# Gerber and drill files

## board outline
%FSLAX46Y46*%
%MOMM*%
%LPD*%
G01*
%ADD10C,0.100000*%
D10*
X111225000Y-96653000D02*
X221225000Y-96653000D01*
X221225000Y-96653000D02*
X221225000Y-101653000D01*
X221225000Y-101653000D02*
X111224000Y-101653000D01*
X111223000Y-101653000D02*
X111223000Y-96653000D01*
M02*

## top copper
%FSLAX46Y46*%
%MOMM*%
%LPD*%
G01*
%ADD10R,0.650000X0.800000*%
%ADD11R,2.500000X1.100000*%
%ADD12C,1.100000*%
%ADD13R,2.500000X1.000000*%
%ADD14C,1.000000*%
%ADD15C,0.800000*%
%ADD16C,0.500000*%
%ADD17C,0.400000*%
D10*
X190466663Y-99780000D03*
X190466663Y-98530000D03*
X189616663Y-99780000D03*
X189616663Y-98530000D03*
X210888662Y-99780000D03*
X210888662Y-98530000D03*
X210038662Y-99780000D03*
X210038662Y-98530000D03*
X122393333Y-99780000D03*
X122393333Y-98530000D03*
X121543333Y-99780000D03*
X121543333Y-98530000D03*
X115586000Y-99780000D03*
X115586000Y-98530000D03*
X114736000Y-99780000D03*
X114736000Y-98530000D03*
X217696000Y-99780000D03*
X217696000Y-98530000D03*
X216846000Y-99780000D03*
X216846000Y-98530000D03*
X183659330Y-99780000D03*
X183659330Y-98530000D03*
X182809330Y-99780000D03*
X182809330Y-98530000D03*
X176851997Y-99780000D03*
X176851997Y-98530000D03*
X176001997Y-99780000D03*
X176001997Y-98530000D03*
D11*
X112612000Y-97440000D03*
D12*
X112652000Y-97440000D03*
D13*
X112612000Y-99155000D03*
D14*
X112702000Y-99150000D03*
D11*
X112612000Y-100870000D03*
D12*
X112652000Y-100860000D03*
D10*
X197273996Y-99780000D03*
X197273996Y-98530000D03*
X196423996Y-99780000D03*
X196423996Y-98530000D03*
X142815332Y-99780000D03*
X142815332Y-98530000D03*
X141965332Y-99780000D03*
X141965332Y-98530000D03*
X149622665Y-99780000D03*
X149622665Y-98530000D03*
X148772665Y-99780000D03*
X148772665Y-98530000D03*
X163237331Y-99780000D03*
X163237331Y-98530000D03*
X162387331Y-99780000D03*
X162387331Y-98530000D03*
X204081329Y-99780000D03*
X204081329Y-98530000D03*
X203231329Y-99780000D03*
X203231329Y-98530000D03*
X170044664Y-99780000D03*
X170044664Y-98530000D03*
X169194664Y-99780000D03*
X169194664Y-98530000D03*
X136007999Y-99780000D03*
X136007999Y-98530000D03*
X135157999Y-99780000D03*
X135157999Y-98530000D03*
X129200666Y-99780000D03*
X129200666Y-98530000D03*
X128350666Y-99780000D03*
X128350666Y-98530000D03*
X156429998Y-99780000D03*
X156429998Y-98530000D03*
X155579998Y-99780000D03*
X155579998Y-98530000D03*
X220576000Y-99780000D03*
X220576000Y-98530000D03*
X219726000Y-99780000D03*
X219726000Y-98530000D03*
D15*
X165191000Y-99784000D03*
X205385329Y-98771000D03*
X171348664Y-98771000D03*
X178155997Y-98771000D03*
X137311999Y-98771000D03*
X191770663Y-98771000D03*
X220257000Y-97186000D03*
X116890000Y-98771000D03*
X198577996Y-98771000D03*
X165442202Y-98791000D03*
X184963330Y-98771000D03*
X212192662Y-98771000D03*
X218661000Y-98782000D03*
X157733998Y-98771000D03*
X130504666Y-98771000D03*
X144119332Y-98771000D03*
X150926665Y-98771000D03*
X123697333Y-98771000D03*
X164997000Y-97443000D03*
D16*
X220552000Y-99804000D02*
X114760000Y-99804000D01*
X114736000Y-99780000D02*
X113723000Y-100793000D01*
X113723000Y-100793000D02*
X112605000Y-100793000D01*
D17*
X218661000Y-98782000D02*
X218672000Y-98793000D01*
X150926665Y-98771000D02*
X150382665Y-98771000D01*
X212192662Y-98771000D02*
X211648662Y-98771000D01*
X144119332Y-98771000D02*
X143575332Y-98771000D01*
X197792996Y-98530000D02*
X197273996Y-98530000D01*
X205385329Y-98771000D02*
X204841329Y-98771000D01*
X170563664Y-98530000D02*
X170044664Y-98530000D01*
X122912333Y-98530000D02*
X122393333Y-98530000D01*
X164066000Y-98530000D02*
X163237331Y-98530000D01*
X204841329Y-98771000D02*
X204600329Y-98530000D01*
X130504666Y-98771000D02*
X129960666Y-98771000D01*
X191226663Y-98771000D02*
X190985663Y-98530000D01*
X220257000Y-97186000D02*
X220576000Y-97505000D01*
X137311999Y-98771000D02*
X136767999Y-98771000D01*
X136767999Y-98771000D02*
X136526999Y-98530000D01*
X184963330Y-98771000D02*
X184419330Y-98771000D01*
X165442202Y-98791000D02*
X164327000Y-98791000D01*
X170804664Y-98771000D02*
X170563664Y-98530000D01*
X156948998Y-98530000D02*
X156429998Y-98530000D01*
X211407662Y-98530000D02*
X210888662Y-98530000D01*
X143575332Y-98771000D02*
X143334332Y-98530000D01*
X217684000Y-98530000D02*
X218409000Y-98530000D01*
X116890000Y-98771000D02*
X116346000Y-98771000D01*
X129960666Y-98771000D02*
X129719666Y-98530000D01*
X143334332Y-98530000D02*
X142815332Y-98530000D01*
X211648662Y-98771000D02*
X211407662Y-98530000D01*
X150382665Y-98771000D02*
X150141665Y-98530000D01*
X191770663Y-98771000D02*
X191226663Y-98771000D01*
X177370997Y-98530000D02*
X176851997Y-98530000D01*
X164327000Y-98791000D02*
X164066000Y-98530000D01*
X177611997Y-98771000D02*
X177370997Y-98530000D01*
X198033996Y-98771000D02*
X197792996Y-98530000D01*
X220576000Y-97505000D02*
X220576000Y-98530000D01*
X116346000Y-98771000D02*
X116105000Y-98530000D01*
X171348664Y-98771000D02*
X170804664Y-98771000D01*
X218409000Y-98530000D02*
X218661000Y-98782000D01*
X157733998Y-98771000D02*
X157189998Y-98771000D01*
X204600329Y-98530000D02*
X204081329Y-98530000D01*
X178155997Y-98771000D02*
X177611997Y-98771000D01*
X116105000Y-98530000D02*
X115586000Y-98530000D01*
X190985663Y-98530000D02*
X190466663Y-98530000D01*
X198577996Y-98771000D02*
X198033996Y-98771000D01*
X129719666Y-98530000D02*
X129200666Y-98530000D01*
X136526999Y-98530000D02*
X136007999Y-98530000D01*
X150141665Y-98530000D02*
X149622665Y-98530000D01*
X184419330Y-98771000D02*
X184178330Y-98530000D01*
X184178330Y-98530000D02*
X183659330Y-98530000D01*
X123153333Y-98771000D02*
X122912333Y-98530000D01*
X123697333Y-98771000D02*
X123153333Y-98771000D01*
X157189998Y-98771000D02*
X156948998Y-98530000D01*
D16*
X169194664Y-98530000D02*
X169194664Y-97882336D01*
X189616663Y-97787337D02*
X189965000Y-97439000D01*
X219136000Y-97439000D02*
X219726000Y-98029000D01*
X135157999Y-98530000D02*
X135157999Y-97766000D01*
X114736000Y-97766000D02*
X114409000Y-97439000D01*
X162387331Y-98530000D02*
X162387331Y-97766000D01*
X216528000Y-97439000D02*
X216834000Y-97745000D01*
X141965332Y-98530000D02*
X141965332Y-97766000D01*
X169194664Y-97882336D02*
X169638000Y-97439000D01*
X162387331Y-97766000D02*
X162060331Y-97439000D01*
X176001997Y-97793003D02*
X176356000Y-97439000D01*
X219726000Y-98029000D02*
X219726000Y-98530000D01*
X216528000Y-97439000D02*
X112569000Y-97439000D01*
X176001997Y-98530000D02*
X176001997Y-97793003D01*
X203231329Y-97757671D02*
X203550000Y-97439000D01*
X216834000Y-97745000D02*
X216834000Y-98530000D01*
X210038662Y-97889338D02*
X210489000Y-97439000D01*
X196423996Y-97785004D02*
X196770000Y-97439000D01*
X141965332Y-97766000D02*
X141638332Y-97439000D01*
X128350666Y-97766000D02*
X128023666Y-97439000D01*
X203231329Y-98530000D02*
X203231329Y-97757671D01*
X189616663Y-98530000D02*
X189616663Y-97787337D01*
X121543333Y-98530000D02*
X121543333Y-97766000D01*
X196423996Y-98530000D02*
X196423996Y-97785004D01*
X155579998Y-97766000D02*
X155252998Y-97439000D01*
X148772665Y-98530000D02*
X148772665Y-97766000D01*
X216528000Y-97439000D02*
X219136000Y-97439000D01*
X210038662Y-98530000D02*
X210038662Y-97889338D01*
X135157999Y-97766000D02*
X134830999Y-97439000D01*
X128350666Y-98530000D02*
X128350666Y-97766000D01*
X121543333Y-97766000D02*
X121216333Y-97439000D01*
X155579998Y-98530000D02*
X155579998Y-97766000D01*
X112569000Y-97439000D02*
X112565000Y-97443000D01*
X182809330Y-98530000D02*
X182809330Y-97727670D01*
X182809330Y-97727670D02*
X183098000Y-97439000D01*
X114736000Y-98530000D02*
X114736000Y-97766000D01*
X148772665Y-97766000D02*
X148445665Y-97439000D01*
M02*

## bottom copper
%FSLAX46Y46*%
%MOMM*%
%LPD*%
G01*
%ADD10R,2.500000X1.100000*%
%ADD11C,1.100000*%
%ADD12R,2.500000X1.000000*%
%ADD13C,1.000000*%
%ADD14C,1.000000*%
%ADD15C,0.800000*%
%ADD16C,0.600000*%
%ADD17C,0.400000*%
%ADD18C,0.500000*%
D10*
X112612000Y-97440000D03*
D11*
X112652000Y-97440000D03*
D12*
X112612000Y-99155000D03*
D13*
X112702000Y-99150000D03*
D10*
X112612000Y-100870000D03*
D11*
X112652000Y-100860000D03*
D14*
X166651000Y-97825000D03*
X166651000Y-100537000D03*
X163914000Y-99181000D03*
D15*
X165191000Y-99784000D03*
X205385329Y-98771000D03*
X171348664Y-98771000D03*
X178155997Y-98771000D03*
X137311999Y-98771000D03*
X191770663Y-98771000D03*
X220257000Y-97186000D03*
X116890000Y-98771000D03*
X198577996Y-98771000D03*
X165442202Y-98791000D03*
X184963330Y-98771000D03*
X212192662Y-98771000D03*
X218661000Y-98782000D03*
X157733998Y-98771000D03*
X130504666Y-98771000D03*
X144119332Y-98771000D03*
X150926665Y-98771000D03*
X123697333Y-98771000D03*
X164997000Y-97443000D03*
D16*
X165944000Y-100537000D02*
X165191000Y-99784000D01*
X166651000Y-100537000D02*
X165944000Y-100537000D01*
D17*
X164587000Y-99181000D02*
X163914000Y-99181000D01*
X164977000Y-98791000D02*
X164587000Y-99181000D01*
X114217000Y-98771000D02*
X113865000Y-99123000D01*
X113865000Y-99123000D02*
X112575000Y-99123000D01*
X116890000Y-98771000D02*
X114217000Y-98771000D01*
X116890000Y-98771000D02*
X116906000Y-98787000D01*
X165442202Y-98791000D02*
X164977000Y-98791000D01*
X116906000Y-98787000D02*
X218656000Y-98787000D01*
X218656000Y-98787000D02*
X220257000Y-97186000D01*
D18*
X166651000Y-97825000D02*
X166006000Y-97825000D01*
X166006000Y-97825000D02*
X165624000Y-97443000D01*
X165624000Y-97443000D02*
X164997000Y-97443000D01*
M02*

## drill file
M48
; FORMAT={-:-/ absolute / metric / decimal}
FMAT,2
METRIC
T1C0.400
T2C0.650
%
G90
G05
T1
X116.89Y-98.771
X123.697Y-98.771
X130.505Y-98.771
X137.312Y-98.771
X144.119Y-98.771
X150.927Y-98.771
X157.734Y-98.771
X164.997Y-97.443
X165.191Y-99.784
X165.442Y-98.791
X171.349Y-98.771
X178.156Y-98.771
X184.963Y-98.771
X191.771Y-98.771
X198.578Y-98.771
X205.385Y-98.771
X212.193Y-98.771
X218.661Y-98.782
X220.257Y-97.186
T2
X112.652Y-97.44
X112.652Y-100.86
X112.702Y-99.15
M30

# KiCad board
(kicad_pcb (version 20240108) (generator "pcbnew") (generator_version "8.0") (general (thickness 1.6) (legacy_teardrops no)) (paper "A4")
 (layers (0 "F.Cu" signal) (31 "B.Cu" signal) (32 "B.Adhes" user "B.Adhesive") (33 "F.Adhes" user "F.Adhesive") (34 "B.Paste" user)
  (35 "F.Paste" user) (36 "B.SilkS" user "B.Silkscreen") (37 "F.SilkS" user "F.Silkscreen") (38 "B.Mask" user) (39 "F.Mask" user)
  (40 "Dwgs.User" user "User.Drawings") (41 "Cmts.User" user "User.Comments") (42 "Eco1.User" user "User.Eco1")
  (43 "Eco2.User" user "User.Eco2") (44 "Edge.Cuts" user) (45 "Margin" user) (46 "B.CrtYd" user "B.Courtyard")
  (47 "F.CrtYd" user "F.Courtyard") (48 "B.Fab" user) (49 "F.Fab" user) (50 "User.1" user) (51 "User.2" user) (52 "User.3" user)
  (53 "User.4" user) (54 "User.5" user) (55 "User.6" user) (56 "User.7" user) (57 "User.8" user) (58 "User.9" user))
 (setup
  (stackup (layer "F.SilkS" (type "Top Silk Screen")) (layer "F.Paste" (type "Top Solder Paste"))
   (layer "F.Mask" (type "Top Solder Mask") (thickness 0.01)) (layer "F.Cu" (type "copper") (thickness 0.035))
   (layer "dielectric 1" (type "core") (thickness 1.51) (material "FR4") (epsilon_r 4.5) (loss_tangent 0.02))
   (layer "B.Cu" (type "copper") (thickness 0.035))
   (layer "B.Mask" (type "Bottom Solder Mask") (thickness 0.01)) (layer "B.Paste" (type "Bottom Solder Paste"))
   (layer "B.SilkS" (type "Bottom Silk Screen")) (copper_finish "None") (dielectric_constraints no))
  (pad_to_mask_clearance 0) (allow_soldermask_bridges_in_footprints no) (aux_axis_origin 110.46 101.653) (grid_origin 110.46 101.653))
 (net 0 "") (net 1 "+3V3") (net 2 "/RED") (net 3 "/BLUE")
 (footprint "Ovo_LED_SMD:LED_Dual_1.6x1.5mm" (layer "F.Cu") (at 190.041663 99.155 90)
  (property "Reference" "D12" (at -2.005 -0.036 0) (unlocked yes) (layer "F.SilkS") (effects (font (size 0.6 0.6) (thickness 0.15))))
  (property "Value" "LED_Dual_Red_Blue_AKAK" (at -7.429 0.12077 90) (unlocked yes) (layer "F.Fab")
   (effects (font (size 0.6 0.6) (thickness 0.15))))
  (pad "1" smd rect (at -0.625 0.425 90) (size 0.8 0.65) (layers "F.Cu" "F.Paste" "F.Mask") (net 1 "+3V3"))
  (pad "2" smd rect (at 0.625 0.425 90) (size 0.8 0.65) (layers "F.Cu" "F.Paste" "F.Mask") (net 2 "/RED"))
  (pad "3" smd rect (at -0.625 -0.425 90) (size 0.8 0.65) (layers "F.Cu" "F.Paste" "F.Mask") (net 1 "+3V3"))
  (pad "4" smd rect (at 0.625 -0.425 90) (size 0.8 0.65) (layers "F.Cu" "F.Paste" "F.Mask") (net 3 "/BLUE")))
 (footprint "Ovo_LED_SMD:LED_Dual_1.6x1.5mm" (layer "F.Cu") (at 210.463662 99.155 90)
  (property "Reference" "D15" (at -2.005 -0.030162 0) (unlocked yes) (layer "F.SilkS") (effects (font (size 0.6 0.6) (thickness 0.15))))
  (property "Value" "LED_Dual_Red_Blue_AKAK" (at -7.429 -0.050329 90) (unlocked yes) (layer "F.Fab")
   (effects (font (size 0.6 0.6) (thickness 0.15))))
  (pad "1" smd rect (at -0.625 0.425 90) (size 0.8 0.65) (layers "F.Cu" "F.Paste" "F.Mask") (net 1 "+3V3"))
  (pad "2" smd rect (at 0.625 0.425 90) (size 0.8 0.65) (layers "F.Cu" "F.Paste" "F.Mask") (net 2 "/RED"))
  (pad "3" smd rect (at -0.625 -0.425 90) (size 0.8 0.65) (layers "F.Cu" "F.Paste" "F.Mask") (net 1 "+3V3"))
  (pad "4" smd rect (at 0.625 -0.425 90) (size 0.8 0.65) (layers "F.Cu" "F.Paste" "F.Mask") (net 3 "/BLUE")))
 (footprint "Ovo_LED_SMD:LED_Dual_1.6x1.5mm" (layer "F.Cu") (at 121.968333 99.155 90)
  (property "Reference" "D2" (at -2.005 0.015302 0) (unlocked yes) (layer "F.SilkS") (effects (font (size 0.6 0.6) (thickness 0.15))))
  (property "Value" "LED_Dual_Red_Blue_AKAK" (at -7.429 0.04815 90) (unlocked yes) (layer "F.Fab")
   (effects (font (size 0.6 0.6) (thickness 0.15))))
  (pad "1" smd rect (at -0.625 0.425 90) (size 0.8 0.65) (layers "F.Cu" "F.Paste" "F.Mask") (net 1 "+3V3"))
  (pad "2" smd rect (at 0.625 0.425 90) (size 0.8 0.65) (layers "F.Cu" "F.Paste" "F.Mask") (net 2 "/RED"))
  (pad "3" smd rect (at -0.625 -0.425 90) (size 0.8 0.65) (layers "F.Cu" "F.Paste" "F.Mask") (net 1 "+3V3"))
  (pad "4" smd rect (at 0.625 -0.425 90) (size 0.8 0.65) (layers "F.Cu" "F.Paste" "F.Mask") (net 3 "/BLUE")))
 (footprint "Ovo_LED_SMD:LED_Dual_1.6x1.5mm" (layer "F.Cu") (at 115.161 99.155 90)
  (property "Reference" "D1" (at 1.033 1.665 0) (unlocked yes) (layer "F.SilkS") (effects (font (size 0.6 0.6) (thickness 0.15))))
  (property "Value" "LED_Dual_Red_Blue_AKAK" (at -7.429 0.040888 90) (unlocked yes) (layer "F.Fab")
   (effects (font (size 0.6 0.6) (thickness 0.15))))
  (pad "1" smd rect (at -0.625 0.425 90) (size 0.8 0.65) (layers "F.Cu" "F.Paste" "F.Mask") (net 1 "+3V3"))
  (pad "2" smd rect (at 0.625 0.425 90) (size 0.8 0.65) (layers "F.Cu" "F.Paste" "F.Mask") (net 2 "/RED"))
  (pad "3" smd rect (at -0.625 -0.425 90) (size 0.8 0.65) (layers "F.Cu" "F.Paste" "F.Mask") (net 1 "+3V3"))
  (pad "4" smd rect (at 0.625 -0.425 90) (size 0.8 0.65) (layers "F.Cu" "F.Paste" "F.Mask") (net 3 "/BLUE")))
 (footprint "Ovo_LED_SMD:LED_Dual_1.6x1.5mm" (layer "F.Cu") (at 217.271 99.155 90)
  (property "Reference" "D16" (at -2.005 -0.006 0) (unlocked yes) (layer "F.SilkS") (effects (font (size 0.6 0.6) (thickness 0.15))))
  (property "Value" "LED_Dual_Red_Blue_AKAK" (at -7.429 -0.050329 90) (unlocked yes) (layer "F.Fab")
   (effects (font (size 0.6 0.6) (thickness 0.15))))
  (pad "1" smd rect (at -0.625 0.425 90) (size 0.8 0.65) (layers "F.Cu" "F.Paste" "F.Mask") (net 1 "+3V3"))
  (pad "2" smd rect (at 0.625 0.425 90) (size 0.8 0.65) (layers "F.Cu" "F.Paste" "F.Mask") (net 2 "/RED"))
  (pad "3" smd rect (at -0.625 -0.425 90) (size 0.8 0.65) (layers "F.Cu" "F.Paste" "F.Mask") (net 1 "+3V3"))
  (pad "4" smd rect (at 0.625 -0.425 90) (size 0.8 0.65) (layers "F.Cu" "F.Paste" "F.Mask") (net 3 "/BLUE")))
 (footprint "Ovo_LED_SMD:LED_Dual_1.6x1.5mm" (layer "F.Cu") (at 183.23433 99.155 90)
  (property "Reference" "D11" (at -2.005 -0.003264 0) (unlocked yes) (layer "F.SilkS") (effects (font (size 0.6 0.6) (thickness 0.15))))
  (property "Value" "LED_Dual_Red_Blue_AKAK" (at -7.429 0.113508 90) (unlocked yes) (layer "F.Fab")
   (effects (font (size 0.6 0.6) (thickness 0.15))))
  (pad "1" smd rect (at -0.625 0.425 90) (size 0.8 0.65) (layers "F.Cu" "F.Paste" "F.Mask") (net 1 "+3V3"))
  (pad "2" smd rect (at 0.625 0.425 90) (size 0.8 0.65) (layers "F.Cu" "F.Paste" "F.Mask") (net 2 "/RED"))
  (pad "3" smd rect (at -0.625 -0.425 90) (size 0.8 0.65) (layers "F.Cu" "F.Paste" "F.Mask") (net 1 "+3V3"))
  (pad "4" smd rect (at 0.625 -0.425 90) (size 0.8 0.65) (layers "F.Cu" "F.Paste" "F.Mask") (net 3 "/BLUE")))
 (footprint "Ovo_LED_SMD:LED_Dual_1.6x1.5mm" (layer "F.Cu") (at 176.426997 99.155 90)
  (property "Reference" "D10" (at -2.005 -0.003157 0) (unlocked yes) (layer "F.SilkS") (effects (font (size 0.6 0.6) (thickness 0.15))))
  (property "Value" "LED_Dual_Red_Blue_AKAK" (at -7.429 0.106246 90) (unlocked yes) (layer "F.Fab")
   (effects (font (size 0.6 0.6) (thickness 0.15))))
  (pad "1" smd rect (at -0.625 0.425 90) (size 0.8 0.65) (layers "F.Cu" "F.Paste" "F.Mask") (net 1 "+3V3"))
  (pad "2" smd rect (at 0.625 0.425 90) (size 0.8 0.65) (layers "F.Cu" "F.Paste" "F.Mask") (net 2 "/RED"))
  (pad "3" smd rect (at -0.625 -0.425 90) (size 0.8 0.65) (layers "F.Cu" "F.Paste" "F.Mask") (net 1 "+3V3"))
  (pad "4" smd rect (at 0.625 -0.425 90) (size 0.8 0.65) (layers "F.Cu" "F.Paste" "F.Mask") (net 3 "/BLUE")))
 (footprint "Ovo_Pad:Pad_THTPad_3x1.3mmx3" (layer "F.Cu") (at 112.652 97.52)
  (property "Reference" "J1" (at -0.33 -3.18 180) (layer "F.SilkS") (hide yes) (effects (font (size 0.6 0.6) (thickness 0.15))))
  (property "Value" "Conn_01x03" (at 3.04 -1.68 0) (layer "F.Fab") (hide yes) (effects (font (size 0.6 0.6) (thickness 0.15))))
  (pad "1" smd rect (at -0.04 -0.08 180) (size 2.5 1.1) (layers "F.Cu" "F.Paste" "F.Mask") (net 3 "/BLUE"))
  (pad "1" smd rect (at -0.04 -0.08 180) (size 2.5 1.1) (layers "B.Cu" "B.Paste" "B.Mask") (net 3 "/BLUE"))
  (pad "1" thru_hole circle (at 0 -0.08) (size 1.1 1.1) (drill 0.65) (layers "*.Cu" "*.Mask") (remove_unused_layers no) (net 3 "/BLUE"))
  (pad "2" smd rect (at -0.04 1.635 180) (size 2.5 1) (layers "F.Cu" "F.Paste" "F.Mask") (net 2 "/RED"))
  (pad "2" smd rect (at -0.04 1.635 180) (size 2.5 1) (layers "B.Cu" "B.Paste" "B.Mask") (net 2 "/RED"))
  (pad "2" thru_hole circle (at 0.05 1.63) (size 1 1) (drill 0.65) (layers "*.Cu" "*.Mask") (remove_unused_layers no) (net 2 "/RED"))
  (pad "3" smd rect (at -0.04 3.35 180) (size 2.5 1.1) (layers "F.Cu" "F.Paste" "F.Mask") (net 1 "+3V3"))
  (pad "3" smd rect (at -0.04 3.35 180) (size 2.5 1.1) (layers "B.Cu" "B.Paste" "B.Mask") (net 1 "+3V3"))
  (pad "3" thru_hole circle (at 0 3.34) (size 1.1 1.1) (drill 0.65) (layers "*.Cu" "*.Mask") (remove_unused_layers no) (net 1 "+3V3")))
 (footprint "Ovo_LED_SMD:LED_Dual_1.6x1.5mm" (layer "F.Cu") (at 196.848996 99.155 90)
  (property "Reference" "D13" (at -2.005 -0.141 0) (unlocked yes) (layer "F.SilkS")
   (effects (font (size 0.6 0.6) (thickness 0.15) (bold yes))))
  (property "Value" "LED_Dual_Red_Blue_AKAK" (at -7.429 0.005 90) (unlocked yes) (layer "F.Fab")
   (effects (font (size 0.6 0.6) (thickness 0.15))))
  (pad "1" smd rect (at -0.625 0.425 90) (size 0.8 0.65) (layers "F.Cu" "F.Paste" "F.Mask") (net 1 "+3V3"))
  (pad "2" smd rect (at 0.625 0.425 90) (size 0.8 0.65) (layers "F.Cu" "F.Paste" "F.Mask") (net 2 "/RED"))
  (pad "3" smd rect (at -0.625 -0.425 90) (size 0.8 0.65) (layers "F.Cu" "F.Paste" "F.Mask") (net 1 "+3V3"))
  (pad "4" smd rect (at 0.625 -0.425 90) (size 0.8 0.65) (layers "F.Cu" "F.Paste" "F.Mask") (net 3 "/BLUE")))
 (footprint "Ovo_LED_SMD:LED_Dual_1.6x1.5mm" (layer "F.Cu") (at 142.390332 99.155 90)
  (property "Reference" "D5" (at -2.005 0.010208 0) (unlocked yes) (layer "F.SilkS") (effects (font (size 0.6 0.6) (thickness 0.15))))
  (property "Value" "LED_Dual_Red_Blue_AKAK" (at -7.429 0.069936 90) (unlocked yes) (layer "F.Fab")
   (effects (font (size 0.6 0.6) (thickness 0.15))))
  (pad "1" smd rect (at -0.625 0.425 90) (size 0.8 0.65) (layers "F.Cu" "F.Paste" "F.Mask") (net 1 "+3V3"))
  (pad "2" smd rect (at 0.625 0.425 90) (size 0.8 0.65) (layers "F.Cu" "F.Paste" "F.Mask") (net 2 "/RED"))
  (pad "3" smd rect (at -0.625 -0.425 90) (size 0.8 0.65) (layers "F.Cu" "F.Paste" "F.Mask") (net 1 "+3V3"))
  (pad "4" smd rect (at 0.625 -0.425 90) (size 0.8 0.65) (layers "F.Cu" "F.Paste" "F.Mask") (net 3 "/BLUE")))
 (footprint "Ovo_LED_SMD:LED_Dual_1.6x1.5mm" (layer "F.Cu") (at 149.197665 99.155 90)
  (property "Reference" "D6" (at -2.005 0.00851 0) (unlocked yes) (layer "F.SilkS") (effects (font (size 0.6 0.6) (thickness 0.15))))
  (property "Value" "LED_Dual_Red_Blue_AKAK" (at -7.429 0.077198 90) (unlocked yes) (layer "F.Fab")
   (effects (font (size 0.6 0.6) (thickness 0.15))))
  (pad "1" smd rect (at -0.625 0.425 90) (size 0.8 0.65) (layers "F.Cu" "F.Paste" "F.Mask") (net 1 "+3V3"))
  (pad "2" smd rect (at 0.625 0.425 90) (size 0.8 0.65) (layers "F.Cu" "F.Paste" "F.Mask") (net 2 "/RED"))
  (pad "3" smd rect (at -0.625 -0.425 90) (size 0.8 0.65) (layers "F.Cu" "F.Paste" "F.Mask") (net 1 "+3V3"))
  (pad "4" smd rect (at 0.625 -0.425 90) (size 0.8 0.65) (layers "F.Cu" "F.Paste" "F.Mask") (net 3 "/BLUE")))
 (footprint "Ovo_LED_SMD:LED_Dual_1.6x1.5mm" (layer "F.Cu") (at 162.812331 99.155 90)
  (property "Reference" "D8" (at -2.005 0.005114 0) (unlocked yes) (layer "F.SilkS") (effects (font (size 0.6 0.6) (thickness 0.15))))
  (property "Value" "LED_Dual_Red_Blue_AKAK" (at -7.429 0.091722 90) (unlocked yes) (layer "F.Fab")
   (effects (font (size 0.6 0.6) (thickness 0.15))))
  (pad "1" smd rect (at -0.625 0.425 90) (size 0.8 0.65) (layers "F.Cu" "F.Paste" "F.Mask") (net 1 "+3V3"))
  (pad "2" smd rect (at 0.625 0.425 90) (size 0.8 0.65) (layers "F.Cu" "F.Paste" "F.Mask") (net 2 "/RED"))
  (pad "3" smd rect (at -0.625 -0.425 90) (size 0.8 0.65) (layers "F.Cu" "F.Paste" "F.Mask") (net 1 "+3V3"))
  (pad "4" smd rect (at 0.625 -0.425 90) (size 0.8 0.65) (layers "F.Cu" "F.Paste" "F.Mask") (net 3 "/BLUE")))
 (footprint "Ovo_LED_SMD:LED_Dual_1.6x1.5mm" (layer "F.Cu") (at 203.656329 99.155 90)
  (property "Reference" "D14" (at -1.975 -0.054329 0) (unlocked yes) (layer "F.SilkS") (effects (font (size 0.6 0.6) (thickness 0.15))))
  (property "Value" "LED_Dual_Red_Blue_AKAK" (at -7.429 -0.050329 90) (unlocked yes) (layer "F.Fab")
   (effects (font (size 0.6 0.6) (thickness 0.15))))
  (pad "1" smd rect (at -0.625 0.425 90) (size 0.8 0.65) (layers "F.Cu" "F.Paste" "F.Mask") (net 1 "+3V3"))
  (pad "2" smd rect (at 0.625 0.425 90) (size 0.8 0.65) (layers "F.Cu" "F.Paste" "F.Mask") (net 2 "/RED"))
  (pad "3" smd rect (at -0.625 -0.425 90) (size 0.8 0.65) (layers "F.Cu" "F.Paste" "F.Mask") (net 1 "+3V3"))
  (pad "4" smd rect (at 0.625 -0.425 90) (size 0.8 0.65) (layers "F.Cu" "F.Paste" "F.Mask") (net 3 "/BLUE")))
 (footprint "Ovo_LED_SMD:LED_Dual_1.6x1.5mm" (layer "F.Cu") (at 169.619664 99.155 90)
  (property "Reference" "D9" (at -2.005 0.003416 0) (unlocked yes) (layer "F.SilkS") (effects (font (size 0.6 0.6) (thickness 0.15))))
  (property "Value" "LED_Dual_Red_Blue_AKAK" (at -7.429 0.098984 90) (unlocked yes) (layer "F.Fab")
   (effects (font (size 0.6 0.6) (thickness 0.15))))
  (pad "1" smd rect (at -0.625 0.425 90) (size 0.8 0.65) (layers "F.Cu" "F.Paste" "F.Mask") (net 1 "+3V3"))
  (pad "2" smd rect (at 0.625 0.425 90) (size 0.8 0.65) (layers "F.Cu" "F.Paste" "F.Mask") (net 2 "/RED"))
  (pad "3" smd rect (at -0.625 -0.425 90) (size 0.8 0.65) (layers "F.Cu" "F.Paste" "F.Mask") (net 1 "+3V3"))
  (pad "4" smd rect (at 0.625 -0.425 90) (size 0.8 0.65) (layers "F.Cu" "F.Paste" "F.Mask") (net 3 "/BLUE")))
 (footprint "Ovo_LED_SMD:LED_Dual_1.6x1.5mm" (layer "F.Cu") (at 135.582999 99.155 90)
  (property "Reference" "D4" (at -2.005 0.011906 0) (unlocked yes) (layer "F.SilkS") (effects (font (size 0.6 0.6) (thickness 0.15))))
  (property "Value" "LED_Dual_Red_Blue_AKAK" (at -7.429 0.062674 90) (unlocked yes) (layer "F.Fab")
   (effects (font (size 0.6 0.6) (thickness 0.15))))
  (pad "1" smd rect (at -0.625 0.425 90) (size 0.8 0.65) (layers "F.Cu" "F.Paste" "F.Mask") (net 1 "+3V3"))
  (pad "2" smd rect (at 0.625 0.425 90) (size 0.8 0.65) (layers "F.Cu" "F.Paste" "F.Mask") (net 2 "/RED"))
  (pad "3" smd rect (at -0.625 -0.425 90) (size 0.8 0.65) (layers "F.Cu" "F.Paste" "F.Mask") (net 1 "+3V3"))
  (pad "4" smd rect (at 0.625 -0.425 90) (size 0.8 0.65) (layers "F.Cu" "F.Paste" "F.Mask") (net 3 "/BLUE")))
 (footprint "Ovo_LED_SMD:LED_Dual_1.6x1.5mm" (layer "F.Cu") (at 128.775666 99.155 90)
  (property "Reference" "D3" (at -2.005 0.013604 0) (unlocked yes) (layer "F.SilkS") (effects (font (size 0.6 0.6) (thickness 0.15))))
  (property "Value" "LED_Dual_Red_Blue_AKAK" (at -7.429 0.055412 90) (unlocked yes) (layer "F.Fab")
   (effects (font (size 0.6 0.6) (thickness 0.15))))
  (pad "1" smd rect (at -0.625 0.425 90) (size 0.8 0.65) (layers "F.Cu" "F.Paste" "F.Mask") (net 1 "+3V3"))
  (pad "2" smd rect (at 0.625 0.425 90) (size 0.8 0.65) (layers "F.Cu" "F.Paste" "F.Mask") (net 2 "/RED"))
  (pad "3" smd rect (at -0.625 -0.425 90) (size 0.8 0.65) (layers "F.Cu" "F.Paste" "F.Mask") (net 1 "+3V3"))
  (pad "4" smd rect (at 0.625 -0.425 90) (size 0.8 0.65) (layers "F.Cu" "F.Paste" "F.Mask") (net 3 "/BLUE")))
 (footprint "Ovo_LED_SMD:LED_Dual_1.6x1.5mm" (layer "F.Cu") (at 156.004998 99.155 90)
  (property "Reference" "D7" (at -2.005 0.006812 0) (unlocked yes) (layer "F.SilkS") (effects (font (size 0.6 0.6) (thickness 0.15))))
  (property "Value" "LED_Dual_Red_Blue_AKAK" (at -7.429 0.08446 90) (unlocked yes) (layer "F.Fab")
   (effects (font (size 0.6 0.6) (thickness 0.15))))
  (pad "1" smd rect (at -0.625 0.425 90) (size 0.8 0.65) (layers "F.Cu" "F.Paste" "F.Mask") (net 1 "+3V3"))
  (pad "2" smd rect (at 0.625 0.425 90) (size 0.8 0.65) (layers "F.Cu" "F.Paste" "F.Mask") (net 2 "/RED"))
  (pad "3" smd rect (at -0.625 -0.425 90) (size 0.8 0.65) (layers "F.Cu" "F.Paste" "F.Mask") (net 1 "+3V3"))
  (pad "4" smd rect (at 0.625 -0.425 90) (size 0.8 0.65) (layers "F.Cu" "F.Paste" "F.Mask") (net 3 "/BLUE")))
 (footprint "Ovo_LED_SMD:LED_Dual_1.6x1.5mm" (layer "F.Cu") (at 220.151 99.155 90)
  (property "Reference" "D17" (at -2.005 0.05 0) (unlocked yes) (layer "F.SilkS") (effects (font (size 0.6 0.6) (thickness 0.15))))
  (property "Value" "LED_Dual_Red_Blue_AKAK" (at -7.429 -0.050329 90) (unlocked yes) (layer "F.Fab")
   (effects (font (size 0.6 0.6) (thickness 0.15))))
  (pad "1" smd rect (at -0.625 0.425 90) (size 0.8 0.65) (layers "F.Cu" "F.Paste" "F.Mask") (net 1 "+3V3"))
  (pad "2" smd rect (at 0.625 0.425 90) (size 0.8 0.65) (layers "F.Cu" "F.Paste" "F.Mask") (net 2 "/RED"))
  (pad "3" smd rect (at -0.625 -0.425 90) (size 0.8 0.65) (layers "F.Cu" "F.Paste" "F.Mask") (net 1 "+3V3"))
  (pad "4" smd rect (at 0.625 -0.425 90) (size 0.8 0.65) (layers "F.Cu" "F.Paste" "F.Mask") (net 3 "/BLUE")))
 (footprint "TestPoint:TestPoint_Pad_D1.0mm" (layer "B.Cu") (at 166.651 97.825 180)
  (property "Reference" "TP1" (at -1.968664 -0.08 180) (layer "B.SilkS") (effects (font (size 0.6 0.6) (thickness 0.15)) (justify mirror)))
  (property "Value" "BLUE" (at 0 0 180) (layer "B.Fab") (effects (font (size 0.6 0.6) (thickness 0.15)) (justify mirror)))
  (pad "1" smd circle (at 0 0 180) (size 1 1) (layers "B.Cu" "B.Mask") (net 3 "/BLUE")))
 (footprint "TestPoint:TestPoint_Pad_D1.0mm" (layer "B.Cu") (at 166.651 100.537 180)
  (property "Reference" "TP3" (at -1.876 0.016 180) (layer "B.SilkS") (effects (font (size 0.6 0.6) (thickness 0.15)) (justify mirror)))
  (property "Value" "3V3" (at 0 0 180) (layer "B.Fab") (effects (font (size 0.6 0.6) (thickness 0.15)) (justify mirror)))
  (pad "1" smd circle (at 0 0 180) (size 1 1) (layers "B.Cu" "B.Mask") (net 1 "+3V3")))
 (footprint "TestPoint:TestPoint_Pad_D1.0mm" (layer "B.Cu") (at 163.914 99.181 180)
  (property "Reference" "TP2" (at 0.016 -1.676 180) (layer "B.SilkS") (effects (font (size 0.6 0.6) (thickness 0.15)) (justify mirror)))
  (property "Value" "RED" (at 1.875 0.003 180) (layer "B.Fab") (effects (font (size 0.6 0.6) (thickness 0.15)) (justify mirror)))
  (pad "1" smd circle (at 0 0 180) (size 1 1) (layers "B.Cu" "B.Mask") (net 2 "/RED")))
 (gr_line (start 111.225 96.653) (end 221.225 96.653) (stroke (width 0.1) (type default)) (layer "Edge.Cuts"))
 (gr_line (start 221.225 96.653) (end 221.225 101.653) (stroke (width 0.1) (type default)) (layer "Edge.Cuts"))
 (gr_line (start 221.225 101.653) (end 111.224 101.653) (stroke (width 0.1) (type default)) (layer "Edge.Cuts"))
 (gr_line (start 111.223 101.653) (end 111.223 96.653) (stroke (width 0.1) (type default)) (layer "Edge.Cuts"))
 (segment (start 220.552 99.804) (end 114.76 99.804) (width 0.5) (layer "F.Cu") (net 1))
 (segment (start 114.736 99.78) (end 113.723 100.793) (width 0.5) (layer "F.Cu") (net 1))
 (segment (start 113.723 100.793) (end 112.605 100.793) (width 0.5) (layer "F.Cu") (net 1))
 (via (at 165.191 99.784) (size 0.8) (drill 0.4) (layers "F.Cu" "B.Cu") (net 1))
 (segment (start 165.944 100.537) (end 165.191 99.784) (width 0.6) (layer "B.Cu") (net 1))
 (segment (start 166.651 100.537) (end 165.944 100.537) (width 0.6) (layer "B.Cu") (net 1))
 (segment (start 218.661 98.782) (end 218.672 98.793) (width 0.4) (layer "F.Cu") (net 2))
 (segment (start 150.926665 98.771) (end 150.382665 98.771) (width 0.4) (layer "F.Cu") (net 2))
 (segment (start 212.192662 98.771) (end 211.648662 98.771) (width 0.4) (layer "F.Cu") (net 2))
 (segment (start 144.119332 98.771) (end 143.575332 98.771) (width 0.4) (layer "F.Cu") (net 2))
 (segment (start 197.792996 98.53) (end 197.273996 98.53) (width 0.4) (layer "F.Cu") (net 2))
 (segment (start 205.385329 98.771) (end 204.841329 98.771) (width 0.4) (layer "F.Cu") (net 2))
 (segment (start 170.563664 98.53) (end 170.044664 98.53) (width 0.4) (layer "F.Cu") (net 2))
 (segment (start 122.912333 98.53) (end 122.393333 98.53) (width 0.4) (layer "F.Cu") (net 2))
 (segment (start 164.066 98.53) (end 163.237331 98.53) (width 0.4) (layer "F.Cu") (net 2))
 (segment (start 204.841329 98.771) (end 204.600329 98.53) (width 0.4) (layer "F.Cu") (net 2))
 (segment (start 130.504666 98.771) (end 129.960666 98.771) (width 0.4) (layer "F.Cu") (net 2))
 (segment (start 191.226663 98.771) (end 190.985663 98.53) (width 0.4) (layer "F.Cu") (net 2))
 (segment (start 220.257 97.186) (end 220.576 97.505) (width 0.4) (layer "F.Cu") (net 2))
 (segment (start 137.311999 98.771) (end 136.767999 98.771) (width 0.4) (layer "F.Cu") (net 2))
 (segment (start 136.767999 98.771) (end 136.526999 98.53) (width 0.4) (layer "F.Cu") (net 2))
 (segment (start 184.96333 98.771) (end 184.41933 98.771) (width 0.4) (layer "F.Cu") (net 2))
 (segment (start 165.442202 98.791) (end 164.327 98.791) (width 0.4) (layer "F.Cu") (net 2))
 (segment (start 170.804664 98.771) (end 170.563664 98.53) (width 0.4) (layer "F.Cu") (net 2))
 (segment (start 156.948998 98.53) (end 156.429998 98.53) (width 0.4) (layer "F.Cu") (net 2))
 (segment (start 211.407662 98.53) (end 210.888662 98.53) (width 0.4) (layer "F.Cu") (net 2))
 (segment (start 143.575332 98.771) (end 143.334332 98.53) (width 0.4) (layer "F.Cu") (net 2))
 (segment (start 217.684 98.53) (end 218.409 98.53) (width 0.4) (layer "F.Cu") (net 2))
 (segment (start 116.89 98.771) (end 116.346 98.771) (width 0.4) (layer "F.Cu") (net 2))
 (segment (start 129.960666 98.771) (end 129.719666 98.53) (width 0.4) (layer "F.Cu") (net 2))
 (segment (start 143.334332 98.53) (end 142.815332 98.53) (width 0.4) (layer "F.Cu") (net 2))
 (segment (start 211.648662 98.771) (end 211.407662 98.53) (width 0.4) (layer "F.Cu") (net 2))
 (segment (start 150.382665 98.771) (end 150.141665 98.53) (width 0.4) (layer "F.Cu") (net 2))
 (segment (start 191.770663 98.771) (end 191.226663 98.771) (width 0.4) (layer "F.Cu") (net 2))
 (segment (start 177.370997 98.53) (end 176.851997 98.53) (width 0.4) (layer "F.Cu") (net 2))
 (segment (start 164.327 98.791) (end 164.066 98.53) (width 0.4) (layer "F.Cu") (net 2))
 (segment (start 177.611997 98.771) (end 177.370997 98.53) (width 0.4) (layer "F.Cu") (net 2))
 (segment (start 198.033996 98.771) (end 197.792996 98.53) (width 0.4) (layer "F.Cu") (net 2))
 (segment (start 220.576 97.505) (end 220.576 98.53) (width 0.4) (layer "F.Cu") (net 2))
 (segment (start 116.346 98.771) (end 116.105 98.53) (width 0.4) (layer "F.Cu") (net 2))
 (segment (start 171.348664 98.771) (end 170.804664 98.771) (width 0.4) (layer "F.Cu") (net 2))
 (segment (start 218.409 98.53) (end 218.661 98.782) (width 0.4) (layer "F.Cu") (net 2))
 (segment (start 157.733998 98.771) (end 157.189998 98.771) (width 0.4) (layer "F.Cu") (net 2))
 (segment (start 204.600329 98.53) (end 204.081329 98.53) (width 0.4) (layer "F.Cu") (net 2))
 (segment (start 178.155997 98.771) (end 177.611997 98.771) (width 0.4) (layer "F.Cu") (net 2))
 (segment (start 116.105 98.53) (end 115.586 98.53) (width 0.4) (layer "F.Cu") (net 2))
 (segment (start 190.985663 98.53) (end 190.466663 98.53) (width 0.4) (layer "F.Cu") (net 2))
 (segment (start 198.577996 98.771) (end 198.033996 98.771) (width 0.4) (layer "F.Cu") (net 2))
 (segment (start 129.719666 98.53) (end 129.200666 98.53) (width 0.4) (layer "F.Cu") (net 2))
 (segment (start 136.526999 98.53) (end 136.007999 98.53) (width 0.4) (layer "F.Cu") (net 2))
 (segment (start 150.141665 98.53) (end 149.622665 98.53) (width 0.4) (layer "F.Cu") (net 2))
 (segment (start 184.41933 98.771) (end 184.17833 98.53) (width 0.4) (layer "F.Cu") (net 2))
 (segment (start 184.17833 98.53) (end 183.65933 98.53) (width 0.4) (layer "F.Cu") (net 2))
 (segment (start 123.153333 98.771) (end 122.912333 98.53) (width 0.4) (layer "F.Cu") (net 2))
 (segment (start 123.697333 98.771) (end 123.153333 98.771) (width 0.4) (layer "F.Cu") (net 2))
 (segment (start 157.189998 98.771) (end 156.948998 98.53) (width 0.4) (layer "F.Cu") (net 2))
 (via (at 205.385329 98.771) (size 0.8) (drill 0.4) (layers "F.Cu" "B.Cu") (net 2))
 (via (at 171.348664 98.771) (size 0.8) (drill 0.4) (layers "F.Cu" "B.Cu") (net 2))
 (via (at 178.155997 98.771) (size 0.8) (drill 0.4) (layers "F.Cu" "B.Cu") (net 2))
 (via (at 137.311999 98.771) (size 0.8) (drill 0.4) (layers "F.Cu" "B.Cu") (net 2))
 (via (at 191.770663 98.771) (size 0.8) (drill 0.4) (layers "F.Cu" "B.Cu") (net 2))
 (via (at 220.257 97.186) (size 0.8) (drill 0.4) (layers "F.Cu" "B.Cu") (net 2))
 (via (at 116.89 98.771) (size 0.8) (drill 0.4) (layers "F.Cu" "B.Cu") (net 2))
 (via (at 198.577996 98.771) (size 0.8) (drill 0.4) (layers "F.Cu" "B.Cu") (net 2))
 (via (at 165.442202 98.791) (size 0.8) (drill 0.4) (layers "F.Cu" "B.Cu") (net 2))
 (via (at 184.96333 98.771) (size 0.8) (drill 0.4) (layers "F.Cu" "B.Cu") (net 2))
 (via (at 212.192662 98.771) (size 0.8) (drill 0.4) (layers "F.Cu" "B.Cu") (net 2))
 (via (at 218.661 98.782) (size 0.8) (drill 0.4) (layers "F.Cu" "B.Cu") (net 2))
 (via (at 157.733998 98.771) (size 0.8) (drill 0.4) (layers "F.Cu" "B.Cu") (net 2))
 (via (at 130.504666 98.771) (size 0.8) (drill 0.4) (layers "F.Cu" "B.Cu") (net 2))
 (via (at 144.119332 98.771) (size 0.8) (drill 0.4) (layers "F.Cu" "B.Cu") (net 2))
 (via (at 150.926665 98.771) (size 0.8) (drill 0.4) (layers "F.Cu" "B.Cu") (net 2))
 (via (at 123.697333 98.771) (size 0.8) (drill 0.4) (layers "F.Cu" "B.Cu") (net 2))
 (segment (start 164.587 99.181) (end 163.914 99.181) (width 0.4) (layer "B.Cu") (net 2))
 (segment (start 164.977 98.791) (end 164.587 99.181) (width 0.4) (layer "B.Cu") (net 2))
 (segment (start 114.217 98.771) (end 113.865 99.123) (width 0.4) (layer "B.Cu") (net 2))
 (segment (start 113.865 99.123) (end 112.575 99.123) (width 0.4) (layer "B.Cu") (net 2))
 (segment (start 116.89 98.771) (end 114.217 98.771) (width 0.4) (layer "B.Cu") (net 2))
 (segment (start 116.89 98.771) (end 116.906 98.787) (width 0.4) (layer "B.Cu") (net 2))
 (segment (start 165.442202 98.791) (end 164.977 98.791) (width 0.4) (layer "B.Cu") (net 2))
 (segment (start 116.906 98.787) (end 218.656 98.787) (width 0.4) (layer "B.Cu") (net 2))
 (segment (start 218.656 98.787) (end 220.257 97.186) (width 0.4) (layer "B.Cu") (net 2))
 (segment (start 169.194664 98.53) (end 169.194664 97.882336) (width 0.5) (layer "F.Cu") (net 3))
 (segment (start 189.616663 97.787337) (end 189.965 97.439) (width 0.5) (layer "F.Cu") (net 3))
 (segment (start 219.136 97.439) (end 219.726 98.029) (width 0.5) (layer "F.Cu") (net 3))
 (segment (start 135.157999 98.53) (end 135.157999 97.766) (width 0.5) (layer "F.Cu") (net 3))
 (segment (start 114.736 97.766) (end 114.409 97.439) (width 0.5) (layer "F.Cu") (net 3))
 (segment (start 162.387331 98.53) (end 162.387331 97.766) (width 0.5) (layer "F.Cu") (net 3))
 (segment (start 216.528 97.439) (end 216.834 97.745) (width 0.5) (layer "F.Cu") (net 3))
 (segment (start 141.965332 98.53) (end 141.965332 97.766) (width 0.5) (layer "F.Cu") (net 3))
 (segment (start 169.194664 97.882336) (end 169.638 97.439) (width 0.5) (layer "F.Cu") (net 3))
 (segment (start 162.387331 97.766) (end 162.060331 97.439) (width 0.5) (layer "F.Cu") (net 3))
 (segment (start 176.001997 97.793003) (end 176.356 97.439) (width 0.5) (layer "F.Cu") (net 3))
 (segment (start 219.726 98.029) (end 219.726 98.53) (width 0.5) (layer "F.Cu") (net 3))
 (segment (start 216.528 97.439) (end 112.569 97.439) (width 0.5) (layer "F.Cu") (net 3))
 (segment (start 176.001997 98.53) (end 176.001997 97.793003) (width 0.5) (layer "F.Cu") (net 3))
 (segment (start 203.231329 97.757671) (end 203.55 97.439) (width 0.5) (layer "F.Cu") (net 3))
 (segment (start 216.834 97.745) (end 216.834 98.53) (width 0.5) (layer "F.Cu") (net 3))
 (segment (start 210.038662 97.889338) (end 210.489 97.439) (width 0.5) (layer "F.Cu") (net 3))
 (segment (start 196.423996 97.785004) (end 196.77 97.439) (width 0.5) (layer "F.Cu") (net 3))
 (segment (start 141.965332 97.766) (end 141.638332 97.439) (width 0.5) (layer "F.Cu") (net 3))
 (segment (start 128.350666 97.766) (end 128.023666 97.439) (width 0.5) (layer "F.Cu") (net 3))
 (segment (start 203.231329 98.53) (end 203.231329 97.757671) (width 0.5) (layer "F.Cu") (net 3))
 (segment (start 189.616663 98.53) (end 189.616663 97.787337) (width 0.5) (layer "F.Cu") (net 3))
 (segment (start 121.543333 98.53) (end 121.543333 97.766) (width 0.5) (layer "F.Cu") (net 3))
 (segment (start 196.423996 98.53) (end 196.423996 97.785004) (width 0.5) (layer "F.Cu") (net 3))
 (segment (start 155.579998 97.766) (end 155.252998 97.439) (width 0.5) (layer "F.Cu") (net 3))
 (segment (start 148.772665 98.53) (end 148.772665 97.766) (width 0.5) (layer "F.Cu") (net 3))
 (segment (start 216.528 97.439) (end 219.136 97.439) (width 0.5) (layer "F.Cu") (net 3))
 (segment (start 210.038662 98.53) (end 210.038662 97.889338) (width 0.5) (layer "F.Cu") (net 3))
 (segment (start 135.157999 97.766) (end 134.830999 97.439) (width 0.5) (layer "F.Cu") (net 3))
 (segment (start 128.350666 98.53) (end 128.350666 97.766) (width 0.5) (layer "F.Cu") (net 3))
 (segment (start 121.543333 97.766) (end 121.216333 97.439) (width 0.5) (layer "F.Cu") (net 3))
 (segment (start 155.579998 98.53) (end 155.579998 97.766) (width 0.5) (layer "F.Cu") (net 3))
 (segment (start 112.569 97.439) (end 112.565 97.443) (width 0.5) (layer "F.Cu") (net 3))
 (segment (start 182.80933 98.53) (end 182.80933 97.72767) (width 0.5) (layer "F.Cu") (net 3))
 (segment (start 182.80933 97.72767) (end 183.098 97.439) (width 0.5) (layer "F.Cu") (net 3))
 (segment (start 114.736 98.53) (end 114.736 97.766) (width 0.5) (layer "F.Cu") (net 3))
 (segment (start 148.772665 97.766) (end 148.445665 97.439) (width 0.5) (layer "F.Cu") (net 3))
 (via (at 164.997 97.443) (size 0.8) (drill 0.4) (layers "F.Cu" "B.Cu") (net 3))
 (segment (start 166.651 97.825) (end 166.006 97.825) (width 0.5) (layer "B.Cu") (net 3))
 (segment (start 166.006 97.825) (end 165.624 97.443) (width 0.5) (layer "B.Cu") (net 3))
 (segment (start 165.624 97.443) (end 164.997 97.443) (width 0.5) (layer "B.Cu") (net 3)))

